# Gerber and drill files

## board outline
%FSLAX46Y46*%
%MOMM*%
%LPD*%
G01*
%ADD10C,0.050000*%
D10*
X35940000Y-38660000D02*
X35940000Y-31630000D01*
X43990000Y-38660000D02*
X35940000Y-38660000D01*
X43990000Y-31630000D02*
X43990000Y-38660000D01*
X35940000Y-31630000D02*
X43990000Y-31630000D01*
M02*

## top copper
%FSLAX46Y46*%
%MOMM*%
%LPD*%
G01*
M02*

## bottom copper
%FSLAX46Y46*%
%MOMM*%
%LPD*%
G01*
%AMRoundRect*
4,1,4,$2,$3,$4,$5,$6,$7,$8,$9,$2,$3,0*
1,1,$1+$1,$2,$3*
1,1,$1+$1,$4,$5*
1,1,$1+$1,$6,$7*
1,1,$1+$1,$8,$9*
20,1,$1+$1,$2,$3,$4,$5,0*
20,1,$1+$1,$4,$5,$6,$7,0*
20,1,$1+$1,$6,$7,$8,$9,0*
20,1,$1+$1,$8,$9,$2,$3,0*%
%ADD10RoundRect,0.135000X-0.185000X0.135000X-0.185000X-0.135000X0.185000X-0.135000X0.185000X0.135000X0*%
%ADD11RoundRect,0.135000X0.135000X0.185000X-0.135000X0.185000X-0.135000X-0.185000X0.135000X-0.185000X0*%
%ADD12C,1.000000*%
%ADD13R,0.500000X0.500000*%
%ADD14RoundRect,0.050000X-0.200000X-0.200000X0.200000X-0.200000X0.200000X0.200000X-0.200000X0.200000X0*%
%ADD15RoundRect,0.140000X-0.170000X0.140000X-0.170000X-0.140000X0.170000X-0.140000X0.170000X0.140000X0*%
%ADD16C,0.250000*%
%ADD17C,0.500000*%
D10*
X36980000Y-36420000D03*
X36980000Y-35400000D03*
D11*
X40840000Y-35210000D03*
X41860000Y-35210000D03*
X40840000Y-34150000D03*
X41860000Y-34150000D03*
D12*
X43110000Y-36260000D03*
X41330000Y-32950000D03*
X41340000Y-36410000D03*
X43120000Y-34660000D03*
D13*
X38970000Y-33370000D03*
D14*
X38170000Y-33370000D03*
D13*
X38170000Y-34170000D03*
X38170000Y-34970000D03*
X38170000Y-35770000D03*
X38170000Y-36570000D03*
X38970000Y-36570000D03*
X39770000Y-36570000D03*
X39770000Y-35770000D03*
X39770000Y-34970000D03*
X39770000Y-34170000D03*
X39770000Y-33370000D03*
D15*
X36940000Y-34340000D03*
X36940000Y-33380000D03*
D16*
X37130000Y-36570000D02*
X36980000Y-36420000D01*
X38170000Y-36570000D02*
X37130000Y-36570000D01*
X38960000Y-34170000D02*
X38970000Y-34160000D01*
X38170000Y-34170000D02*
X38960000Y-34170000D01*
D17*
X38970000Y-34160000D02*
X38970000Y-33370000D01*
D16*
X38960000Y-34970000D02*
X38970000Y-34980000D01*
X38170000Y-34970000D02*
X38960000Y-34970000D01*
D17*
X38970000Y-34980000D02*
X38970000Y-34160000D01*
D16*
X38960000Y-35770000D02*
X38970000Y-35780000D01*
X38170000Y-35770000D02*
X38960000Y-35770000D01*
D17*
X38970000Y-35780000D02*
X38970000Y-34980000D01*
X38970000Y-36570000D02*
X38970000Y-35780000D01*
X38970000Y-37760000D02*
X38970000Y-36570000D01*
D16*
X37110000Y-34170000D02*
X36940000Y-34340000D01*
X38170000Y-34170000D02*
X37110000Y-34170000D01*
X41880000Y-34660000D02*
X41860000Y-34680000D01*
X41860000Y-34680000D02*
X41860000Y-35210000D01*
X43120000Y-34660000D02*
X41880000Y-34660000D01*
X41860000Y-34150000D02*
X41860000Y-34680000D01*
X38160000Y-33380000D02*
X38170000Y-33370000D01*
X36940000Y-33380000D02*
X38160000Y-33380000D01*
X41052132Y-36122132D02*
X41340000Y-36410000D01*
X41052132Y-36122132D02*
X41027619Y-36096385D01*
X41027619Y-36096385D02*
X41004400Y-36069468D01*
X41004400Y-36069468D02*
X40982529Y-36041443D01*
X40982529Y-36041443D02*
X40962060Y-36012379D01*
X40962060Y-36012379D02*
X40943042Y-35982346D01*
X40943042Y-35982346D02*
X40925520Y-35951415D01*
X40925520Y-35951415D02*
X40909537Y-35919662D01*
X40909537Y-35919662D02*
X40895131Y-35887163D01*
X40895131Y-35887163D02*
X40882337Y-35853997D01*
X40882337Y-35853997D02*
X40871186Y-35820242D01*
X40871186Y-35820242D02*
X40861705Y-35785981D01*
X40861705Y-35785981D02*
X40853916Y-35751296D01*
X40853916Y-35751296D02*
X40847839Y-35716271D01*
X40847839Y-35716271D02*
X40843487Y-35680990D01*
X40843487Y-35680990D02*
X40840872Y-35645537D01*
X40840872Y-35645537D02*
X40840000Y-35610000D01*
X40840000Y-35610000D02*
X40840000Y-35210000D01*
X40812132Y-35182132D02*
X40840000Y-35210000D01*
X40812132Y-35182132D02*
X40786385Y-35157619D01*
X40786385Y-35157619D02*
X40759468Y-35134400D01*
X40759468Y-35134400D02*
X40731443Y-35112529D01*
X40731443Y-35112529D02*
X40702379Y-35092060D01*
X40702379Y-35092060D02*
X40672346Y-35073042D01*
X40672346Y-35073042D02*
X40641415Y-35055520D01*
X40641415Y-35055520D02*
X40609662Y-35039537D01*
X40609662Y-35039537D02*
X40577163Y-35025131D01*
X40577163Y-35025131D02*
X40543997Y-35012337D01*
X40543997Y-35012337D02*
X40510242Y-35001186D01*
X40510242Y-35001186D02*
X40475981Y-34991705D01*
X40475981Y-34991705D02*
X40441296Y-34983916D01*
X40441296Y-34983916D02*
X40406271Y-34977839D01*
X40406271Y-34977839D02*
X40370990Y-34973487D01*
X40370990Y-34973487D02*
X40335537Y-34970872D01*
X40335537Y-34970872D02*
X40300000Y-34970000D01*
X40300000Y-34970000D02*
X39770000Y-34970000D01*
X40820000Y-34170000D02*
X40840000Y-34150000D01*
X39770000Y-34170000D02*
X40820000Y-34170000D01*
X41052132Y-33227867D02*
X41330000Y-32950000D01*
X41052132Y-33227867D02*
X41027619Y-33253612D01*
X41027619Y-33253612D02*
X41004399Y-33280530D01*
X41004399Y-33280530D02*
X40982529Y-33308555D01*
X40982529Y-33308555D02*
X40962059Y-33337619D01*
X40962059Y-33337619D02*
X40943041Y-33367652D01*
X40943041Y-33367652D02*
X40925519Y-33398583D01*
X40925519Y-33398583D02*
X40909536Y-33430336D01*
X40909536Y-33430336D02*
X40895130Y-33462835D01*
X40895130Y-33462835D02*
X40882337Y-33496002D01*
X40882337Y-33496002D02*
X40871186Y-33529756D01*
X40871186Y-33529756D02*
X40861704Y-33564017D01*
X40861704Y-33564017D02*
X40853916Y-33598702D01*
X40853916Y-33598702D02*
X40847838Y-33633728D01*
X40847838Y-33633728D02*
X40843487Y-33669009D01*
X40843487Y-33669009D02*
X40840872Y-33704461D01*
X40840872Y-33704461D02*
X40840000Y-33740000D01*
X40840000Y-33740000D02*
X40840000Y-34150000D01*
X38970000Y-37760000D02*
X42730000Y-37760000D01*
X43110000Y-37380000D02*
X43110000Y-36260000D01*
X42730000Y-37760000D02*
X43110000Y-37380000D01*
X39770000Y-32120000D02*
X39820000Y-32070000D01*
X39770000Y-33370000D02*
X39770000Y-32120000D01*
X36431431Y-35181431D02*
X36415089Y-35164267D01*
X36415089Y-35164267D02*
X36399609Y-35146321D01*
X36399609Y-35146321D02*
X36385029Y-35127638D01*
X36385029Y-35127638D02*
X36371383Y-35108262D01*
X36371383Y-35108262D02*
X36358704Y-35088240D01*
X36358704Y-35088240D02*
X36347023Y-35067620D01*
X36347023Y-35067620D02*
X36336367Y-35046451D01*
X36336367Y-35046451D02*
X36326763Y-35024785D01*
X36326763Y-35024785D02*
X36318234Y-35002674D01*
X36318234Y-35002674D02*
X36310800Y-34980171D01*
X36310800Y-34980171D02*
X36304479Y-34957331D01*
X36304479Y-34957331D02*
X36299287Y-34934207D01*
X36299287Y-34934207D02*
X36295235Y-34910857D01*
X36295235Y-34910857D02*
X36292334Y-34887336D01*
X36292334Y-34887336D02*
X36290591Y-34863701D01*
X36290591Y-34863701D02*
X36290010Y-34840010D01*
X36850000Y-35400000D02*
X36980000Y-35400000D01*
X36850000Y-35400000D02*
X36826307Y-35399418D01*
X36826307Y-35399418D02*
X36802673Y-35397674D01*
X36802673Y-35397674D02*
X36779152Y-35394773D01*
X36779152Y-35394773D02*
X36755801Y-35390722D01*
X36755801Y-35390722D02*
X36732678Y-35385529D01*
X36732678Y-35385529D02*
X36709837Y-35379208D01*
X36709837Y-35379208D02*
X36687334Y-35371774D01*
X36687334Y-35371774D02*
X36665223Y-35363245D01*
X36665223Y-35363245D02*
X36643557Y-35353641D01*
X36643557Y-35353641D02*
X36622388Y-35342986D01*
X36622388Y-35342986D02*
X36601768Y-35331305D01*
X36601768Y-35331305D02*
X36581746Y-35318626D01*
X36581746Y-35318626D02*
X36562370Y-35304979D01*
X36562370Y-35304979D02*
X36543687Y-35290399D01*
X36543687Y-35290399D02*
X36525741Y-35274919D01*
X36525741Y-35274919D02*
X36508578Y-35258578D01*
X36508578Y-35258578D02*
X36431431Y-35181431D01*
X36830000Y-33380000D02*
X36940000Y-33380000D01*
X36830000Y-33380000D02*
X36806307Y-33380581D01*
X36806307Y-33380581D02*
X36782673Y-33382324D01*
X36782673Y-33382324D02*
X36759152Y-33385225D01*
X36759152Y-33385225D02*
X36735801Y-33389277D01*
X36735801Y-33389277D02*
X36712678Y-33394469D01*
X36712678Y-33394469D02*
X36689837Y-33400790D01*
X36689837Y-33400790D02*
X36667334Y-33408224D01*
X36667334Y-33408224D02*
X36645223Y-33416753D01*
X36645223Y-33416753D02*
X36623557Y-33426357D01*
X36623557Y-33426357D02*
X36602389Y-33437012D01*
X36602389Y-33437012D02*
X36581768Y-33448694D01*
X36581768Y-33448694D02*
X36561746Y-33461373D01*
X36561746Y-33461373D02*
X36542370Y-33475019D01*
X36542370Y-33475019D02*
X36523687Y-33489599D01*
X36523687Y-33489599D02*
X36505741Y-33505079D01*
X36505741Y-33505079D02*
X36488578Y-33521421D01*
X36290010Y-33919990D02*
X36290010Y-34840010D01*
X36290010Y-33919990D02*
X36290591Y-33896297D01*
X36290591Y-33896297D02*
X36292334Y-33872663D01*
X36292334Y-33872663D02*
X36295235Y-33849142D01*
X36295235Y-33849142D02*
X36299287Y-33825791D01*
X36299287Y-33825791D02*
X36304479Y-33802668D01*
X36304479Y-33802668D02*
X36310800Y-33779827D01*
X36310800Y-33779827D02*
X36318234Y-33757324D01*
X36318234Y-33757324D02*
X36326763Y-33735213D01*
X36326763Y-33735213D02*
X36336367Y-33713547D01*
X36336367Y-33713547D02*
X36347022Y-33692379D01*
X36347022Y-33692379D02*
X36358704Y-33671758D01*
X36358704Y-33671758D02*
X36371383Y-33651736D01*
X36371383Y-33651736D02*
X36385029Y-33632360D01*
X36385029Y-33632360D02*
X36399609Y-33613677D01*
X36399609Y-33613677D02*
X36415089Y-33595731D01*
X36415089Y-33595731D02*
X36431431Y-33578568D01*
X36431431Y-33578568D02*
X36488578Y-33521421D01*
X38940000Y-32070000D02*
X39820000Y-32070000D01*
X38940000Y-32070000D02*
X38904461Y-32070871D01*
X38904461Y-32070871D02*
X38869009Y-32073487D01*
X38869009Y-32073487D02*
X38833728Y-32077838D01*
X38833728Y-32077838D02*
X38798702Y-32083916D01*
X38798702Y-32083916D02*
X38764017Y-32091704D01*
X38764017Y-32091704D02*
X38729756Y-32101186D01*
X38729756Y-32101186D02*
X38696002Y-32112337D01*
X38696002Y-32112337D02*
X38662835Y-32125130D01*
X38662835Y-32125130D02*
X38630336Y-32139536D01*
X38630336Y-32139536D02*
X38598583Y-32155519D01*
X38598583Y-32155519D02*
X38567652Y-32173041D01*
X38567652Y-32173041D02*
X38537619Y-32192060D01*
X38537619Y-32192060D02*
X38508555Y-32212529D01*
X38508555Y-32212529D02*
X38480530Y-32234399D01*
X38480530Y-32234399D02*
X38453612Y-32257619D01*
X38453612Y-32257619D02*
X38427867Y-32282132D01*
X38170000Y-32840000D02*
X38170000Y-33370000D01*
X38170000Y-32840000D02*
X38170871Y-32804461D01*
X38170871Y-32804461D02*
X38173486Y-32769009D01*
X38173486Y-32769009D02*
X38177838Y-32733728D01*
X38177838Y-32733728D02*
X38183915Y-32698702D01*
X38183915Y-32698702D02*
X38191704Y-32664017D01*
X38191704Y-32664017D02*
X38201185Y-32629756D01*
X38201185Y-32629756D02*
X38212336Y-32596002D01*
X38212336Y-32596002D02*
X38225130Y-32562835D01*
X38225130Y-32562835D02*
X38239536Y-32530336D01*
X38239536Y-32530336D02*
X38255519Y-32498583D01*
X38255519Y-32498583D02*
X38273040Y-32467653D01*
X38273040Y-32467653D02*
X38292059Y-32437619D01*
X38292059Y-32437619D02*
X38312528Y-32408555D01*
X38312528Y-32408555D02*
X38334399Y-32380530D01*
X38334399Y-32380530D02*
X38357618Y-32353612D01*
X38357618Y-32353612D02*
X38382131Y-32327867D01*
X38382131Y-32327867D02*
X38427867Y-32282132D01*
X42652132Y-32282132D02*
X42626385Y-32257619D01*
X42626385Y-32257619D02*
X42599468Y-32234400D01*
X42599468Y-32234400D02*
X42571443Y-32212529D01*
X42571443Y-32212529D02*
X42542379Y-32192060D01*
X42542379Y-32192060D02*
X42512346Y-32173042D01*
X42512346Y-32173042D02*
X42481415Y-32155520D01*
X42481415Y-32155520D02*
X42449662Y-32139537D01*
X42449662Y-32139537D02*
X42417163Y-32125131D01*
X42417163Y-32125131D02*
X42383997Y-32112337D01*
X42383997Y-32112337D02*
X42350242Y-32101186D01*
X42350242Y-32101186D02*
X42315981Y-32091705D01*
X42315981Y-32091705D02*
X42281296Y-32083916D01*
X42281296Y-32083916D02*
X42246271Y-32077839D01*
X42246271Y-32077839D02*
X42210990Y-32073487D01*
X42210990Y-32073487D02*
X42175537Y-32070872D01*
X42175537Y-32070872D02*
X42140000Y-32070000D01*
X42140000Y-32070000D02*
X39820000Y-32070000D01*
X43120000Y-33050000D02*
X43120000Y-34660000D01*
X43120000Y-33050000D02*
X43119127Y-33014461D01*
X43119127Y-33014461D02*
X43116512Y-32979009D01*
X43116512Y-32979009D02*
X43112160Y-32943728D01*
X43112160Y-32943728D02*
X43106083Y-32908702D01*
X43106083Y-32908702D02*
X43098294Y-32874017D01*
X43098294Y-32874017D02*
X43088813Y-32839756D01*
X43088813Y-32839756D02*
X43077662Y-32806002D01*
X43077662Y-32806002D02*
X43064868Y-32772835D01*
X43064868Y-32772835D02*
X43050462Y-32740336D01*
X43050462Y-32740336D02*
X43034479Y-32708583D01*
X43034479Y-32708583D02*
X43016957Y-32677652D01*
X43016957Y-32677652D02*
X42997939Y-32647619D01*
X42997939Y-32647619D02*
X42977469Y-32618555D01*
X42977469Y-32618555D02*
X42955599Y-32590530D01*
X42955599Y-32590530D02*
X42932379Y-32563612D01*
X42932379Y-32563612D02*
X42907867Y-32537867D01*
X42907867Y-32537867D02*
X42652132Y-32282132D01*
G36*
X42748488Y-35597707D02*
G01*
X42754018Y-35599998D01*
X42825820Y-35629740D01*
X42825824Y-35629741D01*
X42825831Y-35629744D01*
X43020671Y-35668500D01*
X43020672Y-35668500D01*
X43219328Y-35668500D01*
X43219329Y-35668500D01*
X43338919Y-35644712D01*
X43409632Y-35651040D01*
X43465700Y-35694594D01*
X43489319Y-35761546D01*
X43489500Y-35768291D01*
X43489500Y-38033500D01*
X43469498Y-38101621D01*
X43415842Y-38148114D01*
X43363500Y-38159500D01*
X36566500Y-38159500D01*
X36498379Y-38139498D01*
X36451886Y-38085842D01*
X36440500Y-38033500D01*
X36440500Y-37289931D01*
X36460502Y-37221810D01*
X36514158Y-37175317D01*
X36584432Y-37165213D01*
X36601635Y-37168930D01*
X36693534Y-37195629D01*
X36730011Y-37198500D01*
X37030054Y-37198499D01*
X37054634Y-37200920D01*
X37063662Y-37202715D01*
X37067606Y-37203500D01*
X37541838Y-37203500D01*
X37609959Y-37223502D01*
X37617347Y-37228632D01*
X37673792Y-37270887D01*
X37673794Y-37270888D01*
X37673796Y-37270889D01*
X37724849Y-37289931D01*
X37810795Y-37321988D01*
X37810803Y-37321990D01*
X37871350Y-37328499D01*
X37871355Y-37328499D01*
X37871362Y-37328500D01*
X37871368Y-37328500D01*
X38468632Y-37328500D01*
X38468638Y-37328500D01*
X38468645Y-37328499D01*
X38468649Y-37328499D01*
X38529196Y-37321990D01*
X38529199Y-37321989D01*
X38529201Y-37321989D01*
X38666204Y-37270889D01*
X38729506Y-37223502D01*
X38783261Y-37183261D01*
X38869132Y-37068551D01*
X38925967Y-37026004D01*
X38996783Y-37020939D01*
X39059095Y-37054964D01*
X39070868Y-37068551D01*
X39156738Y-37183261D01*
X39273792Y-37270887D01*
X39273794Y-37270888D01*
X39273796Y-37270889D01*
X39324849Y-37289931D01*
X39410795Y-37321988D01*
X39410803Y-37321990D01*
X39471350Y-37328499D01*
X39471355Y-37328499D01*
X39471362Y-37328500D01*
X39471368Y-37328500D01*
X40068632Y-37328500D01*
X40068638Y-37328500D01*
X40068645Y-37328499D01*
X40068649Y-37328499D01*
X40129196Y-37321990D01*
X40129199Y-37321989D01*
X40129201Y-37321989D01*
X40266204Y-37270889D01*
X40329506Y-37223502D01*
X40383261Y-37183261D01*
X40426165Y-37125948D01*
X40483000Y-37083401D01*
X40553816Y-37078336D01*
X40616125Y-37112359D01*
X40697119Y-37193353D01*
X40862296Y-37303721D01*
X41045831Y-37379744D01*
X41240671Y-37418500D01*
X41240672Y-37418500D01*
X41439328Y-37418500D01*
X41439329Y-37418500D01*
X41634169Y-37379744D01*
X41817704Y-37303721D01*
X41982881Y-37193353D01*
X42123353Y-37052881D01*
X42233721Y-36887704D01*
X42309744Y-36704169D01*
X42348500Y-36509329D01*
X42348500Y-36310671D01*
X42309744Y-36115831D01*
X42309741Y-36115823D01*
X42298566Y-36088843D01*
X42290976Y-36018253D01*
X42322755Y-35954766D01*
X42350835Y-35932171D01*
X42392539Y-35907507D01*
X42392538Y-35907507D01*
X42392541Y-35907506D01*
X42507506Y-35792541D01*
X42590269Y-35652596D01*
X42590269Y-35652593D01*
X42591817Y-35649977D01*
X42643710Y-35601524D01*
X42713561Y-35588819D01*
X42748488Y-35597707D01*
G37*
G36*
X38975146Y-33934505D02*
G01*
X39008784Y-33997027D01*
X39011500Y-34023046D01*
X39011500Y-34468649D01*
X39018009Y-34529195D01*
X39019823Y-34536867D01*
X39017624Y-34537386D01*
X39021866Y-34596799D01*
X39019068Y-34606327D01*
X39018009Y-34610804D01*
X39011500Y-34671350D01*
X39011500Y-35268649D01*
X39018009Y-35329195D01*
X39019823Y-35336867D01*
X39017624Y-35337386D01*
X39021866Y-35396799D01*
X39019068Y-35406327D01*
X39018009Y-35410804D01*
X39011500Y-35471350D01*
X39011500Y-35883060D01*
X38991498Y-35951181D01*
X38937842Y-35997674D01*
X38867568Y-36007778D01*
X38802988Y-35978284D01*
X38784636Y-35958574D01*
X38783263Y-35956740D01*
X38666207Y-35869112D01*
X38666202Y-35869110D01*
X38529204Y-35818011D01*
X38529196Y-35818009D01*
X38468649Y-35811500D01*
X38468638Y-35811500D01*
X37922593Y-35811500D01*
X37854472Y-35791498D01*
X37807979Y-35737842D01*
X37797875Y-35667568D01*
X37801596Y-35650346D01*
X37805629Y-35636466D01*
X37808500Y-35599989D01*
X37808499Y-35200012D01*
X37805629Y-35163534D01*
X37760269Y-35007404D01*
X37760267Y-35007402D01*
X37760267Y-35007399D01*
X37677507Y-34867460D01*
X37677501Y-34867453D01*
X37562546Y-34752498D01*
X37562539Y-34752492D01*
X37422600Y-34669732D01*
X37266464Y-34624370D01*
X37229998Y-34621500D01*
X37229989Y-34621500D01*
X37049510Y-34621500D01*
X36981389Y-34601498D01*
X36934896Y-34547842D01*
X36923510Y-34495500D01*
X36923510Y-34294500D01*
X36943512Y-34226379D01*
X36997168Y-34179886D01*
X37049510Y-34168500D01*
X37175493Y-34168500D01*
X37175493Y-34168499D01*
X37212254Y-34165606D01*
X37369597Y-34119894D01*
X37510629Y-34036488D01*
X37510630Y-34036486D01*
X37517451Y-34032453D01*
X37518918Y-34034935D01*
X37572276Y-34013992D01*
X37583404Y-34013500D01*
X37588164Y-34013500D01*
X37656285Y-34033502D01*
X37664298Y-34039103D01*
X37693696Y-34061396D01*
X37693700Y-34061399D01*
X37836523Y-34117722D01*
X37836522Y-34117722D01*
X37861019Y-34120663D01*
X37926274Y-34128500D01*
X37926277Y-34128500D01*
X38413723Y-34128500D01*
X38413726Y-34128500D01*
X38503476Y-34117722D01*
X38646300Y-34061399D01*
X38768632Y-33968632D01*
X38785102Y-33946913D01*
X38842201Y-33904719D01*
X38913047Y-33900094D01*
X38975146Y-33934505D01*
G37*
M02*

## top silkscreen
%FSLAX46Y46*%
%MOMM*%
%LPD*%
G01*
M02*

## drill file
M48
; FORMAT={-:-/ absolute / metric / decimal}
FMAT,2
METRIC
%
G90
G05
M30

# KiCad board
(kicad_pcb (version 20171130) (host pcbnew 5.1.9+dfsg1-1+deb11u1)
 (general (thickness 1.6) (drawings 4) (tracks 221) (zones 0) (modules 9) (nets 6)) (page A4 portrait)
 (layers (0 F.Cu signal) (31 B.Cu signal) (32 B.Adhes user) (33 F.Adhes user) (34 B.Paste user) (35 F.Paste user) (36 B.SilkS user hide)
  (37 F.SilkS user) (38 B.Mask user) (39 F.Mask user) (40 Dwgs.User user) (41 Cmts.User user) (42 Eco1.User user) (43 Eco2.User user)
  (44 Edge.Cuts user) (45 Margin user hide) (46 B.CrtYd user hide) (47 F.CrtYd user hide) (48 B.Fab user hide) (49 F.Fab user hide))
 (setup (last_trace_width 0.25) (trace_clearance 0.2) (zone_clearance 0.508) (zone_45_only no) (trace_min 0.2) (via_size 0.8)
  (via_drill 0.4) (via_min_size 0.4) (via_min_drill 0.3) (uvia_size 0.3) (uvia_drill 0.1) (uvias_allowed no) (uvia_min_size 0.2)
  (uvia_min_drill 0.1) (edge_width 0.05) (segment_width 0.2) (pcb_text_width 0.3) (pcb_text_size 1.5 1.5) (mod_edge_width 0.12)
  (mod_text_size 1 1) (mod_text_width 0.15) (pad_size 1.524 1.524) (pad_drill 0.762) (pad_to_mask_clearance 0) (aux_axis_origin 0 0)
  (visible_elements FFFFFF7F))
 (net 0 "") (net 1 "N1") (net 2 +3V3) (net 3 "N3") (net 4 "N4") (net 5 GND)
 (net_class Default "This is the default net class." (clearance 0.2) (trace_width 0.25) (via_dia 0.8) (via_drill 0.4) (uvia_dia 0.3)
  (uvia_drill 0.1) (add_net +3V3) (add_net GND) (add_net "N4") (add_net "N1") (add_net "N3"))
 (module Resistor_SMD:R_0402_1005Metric (layer B.Cu) (at 36.98 35.91 270)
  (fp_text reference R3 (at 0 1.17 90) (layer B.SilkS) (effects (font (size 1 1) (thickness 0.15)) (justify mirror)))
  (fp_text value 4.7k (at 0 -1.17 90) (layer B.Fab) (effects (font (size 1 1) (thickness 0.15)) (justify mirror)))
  (pad 2 smd roundrect (at 0.51 0 270) (size 0.54 0.64) (layers B.Cu B.Paste B.Mask) (roundrect_rratio 0.25) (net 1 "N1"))
  (pad 1 smd roundrect (at -0.51 0 270) (size 0.54 0.64) (layers B.Cu B.Paste B.Mask) (roundrect_rratio 0.25) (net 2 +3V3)))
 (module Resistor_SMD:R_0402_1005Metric (layer B.Cu) (at 41.35 35.21 180)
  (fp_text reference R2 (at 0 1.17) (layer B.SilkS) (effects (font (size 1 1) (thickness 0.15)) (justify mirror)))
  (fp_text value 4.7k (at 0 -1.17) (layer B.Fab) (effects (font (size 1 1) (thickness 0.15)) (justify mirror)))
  (pad 2 smd roundrect (at 0.51 0 180) (size 0.54 0.64) (layers B.Cu B.Paste B.Mask) (roundrect_rratio 0.25) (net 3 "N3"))
  (pad 1 smd roundrect (at -0.51 0 180) (size 0.54 0.64) (layers B.Cu B.Paste B.Mask) (roundrect_rratio 0.25) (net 2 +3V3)))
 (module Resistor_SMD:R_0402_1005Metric (layer B.Cu) (at 41.35 34.15 180)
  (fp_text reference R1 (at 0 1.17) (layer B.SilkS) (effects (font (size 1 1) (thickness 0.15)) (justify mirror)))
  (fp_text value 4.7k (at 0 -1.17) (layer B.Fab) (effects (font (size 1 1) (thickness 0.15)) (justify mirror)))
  (pad 2 smd roundrect (at 0.51 0 180) (size 0.54 0.64) (layers B.Cu B.Paste B.Mask) (roundrect_rratio 0.25) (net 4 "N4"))
  (pad 1 smd roundrect (at -0.51 0 180) (size 0.54 0.64) (layers B.Cu B.Paste B.Mask) (roundrect_rratio 0.25) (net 2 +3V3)))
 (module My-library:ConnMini (layer B.Cu) (at 43.11 36.26)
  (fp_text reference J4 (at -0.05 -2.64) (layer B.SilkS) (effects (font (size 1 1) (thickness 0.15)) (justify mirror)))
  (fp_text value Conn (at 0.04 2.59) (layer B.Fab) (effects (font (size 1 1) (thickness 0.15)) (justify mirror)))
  (pad 1 smd circle (at 0 0) (size 1 1) (layers B.Cu B.Paste B.Mask) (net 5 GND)))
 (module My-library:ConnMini (layer B.Cu) (at 41.33 32.95)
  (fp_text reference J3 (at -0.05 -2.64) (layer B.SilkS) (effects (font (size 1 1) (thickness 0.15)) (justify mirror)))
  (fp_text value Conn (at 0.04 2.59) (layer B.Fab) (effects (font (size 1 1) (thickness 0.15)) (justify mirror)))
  (pad 1 smd circle (at 0 0) (size 1 1) (layers B.Cu B.Paste B.Mask) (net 4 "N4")))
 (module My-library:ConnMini (layer B.Cu) (at 41.34 36.41)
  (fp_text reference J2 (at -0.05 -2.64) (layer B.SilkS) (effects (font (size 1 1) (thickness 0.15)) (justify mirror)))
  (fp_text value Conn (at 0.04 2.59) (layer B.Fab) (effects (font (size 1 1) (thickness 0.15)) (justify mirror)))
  (pad 1 smd circle (at 0 0) (size 1 1) (layers B.Cu B.Paste B.Mask) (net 3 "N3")))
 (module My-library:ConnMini (layer B.Cu) (at 43.12 34.66)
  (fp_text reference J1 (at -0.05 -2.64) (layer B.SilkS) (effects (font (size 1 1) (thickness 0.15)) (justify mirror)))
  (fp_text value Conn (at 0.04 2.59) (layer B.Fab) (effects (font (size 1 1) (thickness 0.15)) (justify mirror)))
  (pad 1 smd circle (at 0 0) (size 1 1) (layers B.Cu B.Paste B.Mask) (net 2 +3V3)))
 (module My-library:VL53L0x (layer B.Cu) (at 38.97 34.97)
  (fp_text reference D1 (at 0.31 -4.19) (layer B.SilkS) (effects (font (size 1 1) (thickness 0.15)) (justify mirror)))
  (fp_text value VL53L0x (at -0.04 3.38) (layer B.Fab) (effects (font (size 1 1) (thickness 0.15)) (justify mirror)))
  (pad 12 smd rect (at 0 -1.6) (size 0.5 0.5) (layers B.Cu B.Paste B.Mask) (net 5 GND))
  (pad 1 smd roundrect (at -0.8 -1.6) (size 0.5 0.5) (layers B.Cu B.Paste B.Mask) (roundrect_rratio 0.1) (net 2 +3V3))
  (pad 2 smd rect (at -0.8 -0.8) (size 0.5 0.5) (layers B.Cu B.Paste B.Mask) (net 5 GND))
  (pad 3 smd rect (at -0.8 0) (size 0.5 0.5) (layers B.Cu B.Paste B.Mask) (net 5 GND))
  (pad 4 smd rect (at -0.8 0.8) (size 0.5 0.5) (layers B.Cu B.Paste B.Mask) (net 5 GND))
  (pad 5 smd rect (at -0.8 1.6) (size 0.5 0.5) (layers B.Cu B.Paste B.Mask) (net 1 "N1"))
  (pad 6 smd rect (at 0 1.6) (size 0.5 0.5) (layers B.Cu B.Paste B.Mask) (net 5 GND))
  (pad 7 smd rect (at 0.8 1.6) (size 0.5 0.5) (layers B.Cu B.Paste B.Mask))
  (pad 8 smd rect (at 0.8 0.8) (size 0.5 0.5) (layers B.Cu B.Paste B.Mask))
  (pad 9 smd rect (at 0.8 0) (size 0.5 0.5) (layers B.Cu B.Paste B.Mask) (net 3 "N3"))
  (pad 10 smd rect (at 0.8 -0.8) (size 0.5 0.5) (layers B.Cu B.Paste B.Mask) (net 4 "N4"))
  (pad 11 smd rect (at 0.8 -1.6) (size 0.5 0.5) (layers B.Cu B.Paste B.Mask) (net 2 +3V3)))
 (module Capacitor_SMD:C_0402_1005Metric (layer B.Cu) (at 36.94 33.86 270)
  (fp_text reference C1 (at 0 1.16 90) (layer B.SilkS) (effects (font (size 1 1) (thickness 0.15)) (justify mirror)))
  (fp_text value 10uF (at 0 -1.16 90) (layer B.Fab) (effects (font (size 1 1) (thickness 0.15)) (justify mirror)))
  (pad 2 smd roundrect (at 0.48 0 270) (size 0.56 0.62) (layers B.Cu B.Paste B.Mask) (roundrect_rratio 0.25) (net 5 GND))
  (pad 1 smd roundrect (at -0.48 0 270) (size 0.56 0.62) (layers B.Cu B.Paste B.Mask) (roundrect_rratio 0.25) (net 2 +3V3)))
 (gr_line (start 35.94 38.66) (end 35.94 31.63) (layer Edge.Cuts) (width 0.05))
 (gr_line (start 43.99 38.66) (end 35.94 38.66) (layer Edge.Cuts) (width 0.05))
 (gr_line (start 43.99 31.63) (end 43.99 38.66) (layer Edge.Cuts) (width 0.05))
 (gr_line (start 35.94 31.63) (end 43.99 31.63) (layer Edge.Cuts) (width 0.05))
 (segment (start 37.13 36.57) (end 36.98 36.42) (width 0.25) (layer B.Cu) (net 1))
 (segment (start 38.17 36.57) (end 37.13 36.57) (width 0.25) (layer B.Cu) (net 1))
 (segment (start 38.96 34.17) (end 38.97 34.16) (width 0.25) (layer B.Cu) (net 5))
 (segment (start 38.17 34.17) (end 38.96 34.17) (width 0.25) (layer B.Cu) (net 5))
 (segment (start 38.97 34.16) (end 38.97 33.37) (width 0.5) (layer B.Cu) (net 5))
 (segment (start 38.96 34.97) (end 38.97 34.98) (width 0.25) (layer B.Cu) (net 5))
 (segment (start 38.17 34.97) (end 38.96 34.97) (width 0.25) (layer B.Cu) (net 5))
 (segment (start 38.97 34.98) (end 38.97 34.16) (width 0.5) (layer B.Cu) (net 5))
 (segment (start 38.96 35.77) (end 38.97 35.78) (width 0.25) (layer B.Cu) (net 5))
 (segment (start 38.17 35.77) (end 38.96 35.77) (width 0.25) (layer B.Cu) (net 5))
 (segment (start 38.97 35.78) (end 38.97 34.98) (width 0.5) (layer B.Cu) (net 5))
 (segment (start 38.97 36.57) (end 38.97 35.78) (width 0.5) (layer B.Cu) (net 5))
 (segment (start 38.97 37.76) (end 38.97 36.57) (width 0.5) (layer B.Cu) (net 5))
 (segment (start 37.11 34.17) (end 36.94 34.34) (width 0.25) (layer B.Cu) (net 5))
 (segment (start 38.17 34.17) (end 37.11 34.17) (width 0.25) (layer B.Cu) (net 5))
 (segment (start 41.88 34.66) (end 41.86 34.68) (width 0.25) (layer B.Cu) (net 2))
 (segment (start 41.86 34.68) (end 41.86 35.21) (width 0.25) (layer B.Cu) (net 2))
 (segment (start 43.12 34.66) (end 41.88 34.66) (width 0.25) (layer B.Cu) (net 2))
 (segment (start 41.86 34.15) (end 41.86 34.68) (width 0.25) (layer B.Cu) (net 2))
 (segment (start 38.16 33.38) (end 38.17 33.37) (width 0.25) (layer B.Cu) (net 2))
 (segment (start 36.94 33.38) (end 38.16 33.38) (width 0.25) (layer B.Cu) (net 2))
 (segment (start 41.052132 36.122132) (end 41.34 36.41) (width 0.25) (layer B.Cu) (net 3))
 (segment (start 41.052132 36.122132) (end 41.027619 36.096385) (width 0.25) (layer B.Cu) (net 3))
 (segment (start 41.027619 36.096385) (end 41.0044 36.069468) (width 0.25) (layer B.Cu) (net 3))
 (segment (start 41.0044 36.069468) (end 40.982529 36.041443) (width 0.25) (layer B.Cu) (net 3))
 (segment (start 40.982529 36.041443) (end 40.96206 36.012379) (width 0.25) (layer B.Cu) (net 3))
 (segment (start 40.96206 36.012379) (end 40.943042 35.982346) (width 0.25) (layer B.Cu) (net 3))
 (segment (start 40.943042 35.982346) (end 40.92552 35.951415) (width 0.25) (layer B.Cu) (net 3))
 (segment (start 40.92552 35.951415) (end 40.909537 35.919662) (width 0.25) (layer B.Cu) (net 3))
 (segment (start 40.909537 35.919662) (end 40.895131 35.887163) (width 0.25) (layer B.Cu) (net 3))
 (segment (start 40.895131 35.887163) (end 40.882337 35.853997) (width 0.25) (layer B.Cu) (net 3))
 (segment (start 40.882337 35.853997) (end 40.871186 35.820242) (width 0.25) (layer B.Cu) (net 3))
 (segment (start 40.871186 35.820242) (end 40.861705 35.785981) (width 0.25) (layer B.Cu) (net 3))
 (segment (start 40.861705 35.785981) (end 40.853916 35.751296) (width 0.25) (layer B.Cu) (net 3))
 (segment (start 40.853916 35.751296) (end 40.847839 35.716271) (width 0.25) (layer B.Cu) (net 3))
 (segment (start 40.847839 35.716271) (end 40.843487 35.68099) (width 0.25) (layer B.Cu) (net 3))
 (segment (start 40.843487 35.68099) (end 40.840872 35.645537) (width 0.25) (layer B.Cu) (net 3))
 (segment (start 40.840872 35.645537) (end 40.84 35.61) (width 0.25) (layer B.Cu) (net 3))
 (segment (start 40.84 35.61) (end 40.84 35.21) (width 0.25) (layer B.Cu) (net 3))
 (segment (start 40.812132 35.182132) (end 40.84 35.21) (width 0.25) (layer B.Cu) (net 3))
 (segment (start 40.812132 35.182132) (end 40.786385 35.157619) (width 0.25) (layer B.Cu) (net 3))
 (segment (start 40.786385 35.157619) (end 40.759468 35.1344) (width 0.25) (layer B.Cu) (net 3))
 (segment (start 40.759468 35.1344) (end 40.731443 35.112529) (width 0.25) (layer B.Cu) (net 3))
 (segment (start 40.731443 35.112529) (end 40.702379 35.09206) (width 0.25) (layer B.Cu) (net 3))
 (segment (start 40.702379 35.09206) (end 40.672346 35.073042) (width 0.25) (layer B.Cu) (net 3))
 (segment (start 40.672346 35.073042) (end 40.641415 35.05552) (width 0.25) (layer B.Cu) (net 3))
 (segment (start 40.641415 35.05552) (end 40.609662 35.039537) (width 0.25) (layer B.Cu) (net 3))
 (segment (start 40.609662 35.039537) (end 40.577163 35.025131) (width 0.25) (layer B.Cu) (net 3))
 (segment (start 40.577163 35.025131) (end 40.543997 35.012337) (width 0.25) (layer B.Cu) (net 3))
 (segment (start 40.543997 35.012337) (end 40.510242 35.001186) (width 0.25) (layer B.Cu) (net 3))
 (segment (start 40.510242 35.001186) (end 40.475981 34.991705) (width 0.25) (layer B.Cu) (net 3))
 (segment (start 40.475981 34.991705) (end 40.441296 34.983916) (width 0.25) (layer B.Cu) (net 3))
 (segment (start 40.441296 34.983916) (end 40.406271 34.977839) (width 0.25) (layer B.Cu) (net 3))
 (segment (start 40.406271 34.977839) (end 40.37099 34.973487) (width 0.25) (layer B.Cu) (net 3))
 (segment (start 40.37099 34.973487) (end 40.335537 34.970872) (width 0.25) (layer B.Cu) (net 3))
 (segment (start 40.335537 34.970872) (end 40.3 34.97) (width 0.25) (layer B.Cu) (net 3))
 (segment (start 40.3 34.97) (end 39.77 34.97) (width 0.25) (layer B.Cu) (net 3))
 (segment (start 40.82 34.17) (end 40.84 34.15) (width 0.25) (layer B.Cu) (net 4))
 (segment (start 39.77 34.17) (end 40.82 34.17) (width 0.25) (layer B.Cu) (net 4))
 (segment (start 41.052132 33.227867) (end 41.33 32.95) (width 0.25) (layer B.Cu) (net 4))
 (segment (start 41.052132 33.227867) (end 41.027619 33.253612) (width 0.25) (layer B.Cu) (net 4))
 (segment (start 41.027619 33.253612) (end 41.004399 33.28053) (width 0.25) (layer B.Cu) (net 4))
 (segment (start 41.004399 33.28053) (end 40.982529 33.308555) (width 0.25) (layer B.Cu) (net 4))
 (segment (start 40.982529 33.308555) (end 40.962059 33.337619) (width 0.25) (layer B.Cu) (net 4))
 (segment (start 40.962059 33.337619) (end 40.943041 33.367652) (width 0.25) (layer B.Cu) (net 4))
 (segment (start 40.943041 33.367652) (end 40.925519 33.398583) (width 0.25) (layer B.Cu) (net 4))
 (segment (start 40.925519 33.398583) (end 40.909536 33.430336) (width 0.25) (layer B.Cu) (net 4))
 (segment (start 40.909536 33.430336) (end 40.89513 33.462835) (width 0.25) (layer B.Cu) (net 4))
 (segment (start 40.89513 33.462835) (end 40.882337 33.496002) (width 0.25) (layer B.Cu) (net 4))
 (segment (start 40.882337 33.496002) (end 40.871186 33.529756) (width 0.25) (layer B.Cu) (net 4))
 (segment (start 40.871186 33.529756) (end 40.861704 33.564017) (width 0.25) (layer B.Cu) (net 4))
 (segment (start 40.861704 33.564017) (end 40.853916 33.598702) (width 0.25) (layer B.Cu) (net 4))
 (segment (start 40.853916 33.598702) (end 40.847838 33.633728) (width 0.25) (layer B.Cu) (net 4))
 (segment (start 40.847838 33.633728) (end 40.843487 33.669009) (width 0.25) (layer B.Cu) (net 4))
 (segment (start 40.843487 33.669009) (end 40.840872 33.704461) (width 0.25) (layer B.Cu) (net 4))
 (segment (start 40.840872 33.704461) (end 40.84 33.74) (width 0.25) (layer B.Cu) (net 4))
 (segment (start 40.84 33.74) (end 40.84 34.15) (width 0.25) (layer B.Cu) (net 4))
 (segment (start 38.97 37.76) (end 42.73 37.76) (width 0.25) (layer B.Cu) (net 5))
 (segment (start 43.11 37.38) (end 43.11 36.26) (width 0.25) (layer B.Cu) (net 5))
 (segment (start 42.73 37.76) (end 43.11 37.38) (width 0.25) (layer B.Cu) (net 5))
 (segment (start 39.77 32.12) (end 39.82 32.07) (width 0.25) (layer B.Cu) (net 2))
 (segment (start 39.77 33.37) (end 39.77 32.12) (width 0.25) (layer B.Cu) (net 2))
 (segment (start 36.431431 35.181431) (end 36.415089 35.164267) (width 0.25) (layer B.Cu) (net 2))
 (segment (start 36.415089 35.164267) (end 36.399609 35.146321) (width 0.25) (layer B.Cu) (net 2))
 (segment (start 36.399609 35.146321) (end 36.385029 35.127638) (width 0.25) (layer B.Cu) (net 2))
 (segment (start 36.385029 35.127638) (end 36.371383 35.108262) (width 0.25) (layer B.Cu) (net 2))
 (segment (start 36.371383 35.108262) (end 36.358704 35.08824) (width 0.25) (layer B.Cu) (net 2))
 (segment (start 36.358704 35.08824) (end 36.347023 35.06762) (width 0.25) (layer B.Cu) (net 2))
 (segment (start 36.347023 35.06762) (end 36.336367 35.046451) (width 0.25) (layer B.Cu) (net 2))
 (segment (start 36.336367 35.046451) (end 36.326763 35.024785) (width 0.25) (layer B.Cu) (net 2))
 (segment (start 36.326763 35.024785) (end 36.318234 35.002674) (width 0.25) (layer B.Cu) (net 2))
 (segment (start 36.318234 35.002674) (end 36.3108 34.980171) (width 0.25) (layer B.Cu) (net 2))
 (segment (start 36.3108 34.980171) (end 36.304479 34.957331) (width 0.25) (layer B.Cu) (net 2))
 (segment (start 36.304479 34.957331) (end 36.299287 34.934207) (width 0.25) (layer B.Cu) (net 2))
 (segment (start 36.299287 34.934207) (end 36.295235 34.910857) (width 0.25) (layer B.Cu) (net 2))
 (segment (start 36.295235 34.910857) (end 36.292334 34.887336) (width 0.25) (layer B.Cu) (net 2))
 (segment (start 36.292334 34.887336) (end 36.290591 34.863701) (width 0.25) (layer B.Cu) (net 2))
 (segment (start 36.290591 34.863701) (end 36.29001 34.84001) (width 0.25) (layer B.Cu) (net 2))
 (segment (start 36.85 35.4) (end 36.98 35.4) (width 0.25) (layer B.Cu) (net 2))
 (segment (start 36.85 35.4) (end 36.826307 35.399418) (width 0.25) (layer B.Cu) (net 2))
 (segment (start 36.826307 35.399418) (end 36.802673 35.397674) (width 0.25) (layer B.Cu) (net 2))
 (segment (start 36.802673 35.397674) (end 36.779152 35.394773) (width 0.25) (layer B.Cu) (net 2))
 (segment (start 36.779152 35.394773) (end 36.755801 35.390722) (width 0.25) (layer B.Cu) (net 2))
 (segment (start 36.755801 35.390722) (end 36.732678 35.385529) (width 0.25) (layer B.Cu) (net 2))
 (segment (start 36.732678 35.385529) (end 36.709837 35.379208) (width 0.25) (layer B.Cu) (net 2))
 (segment (start 36.709837 35.379208) (end 36.687334 35.371774) (width 0.25) (layer B.Cu) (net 2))
 (segment (start 36.687334 35.371774) (end 36.665223 35.363245) (width 0.25) (layer B.Cu) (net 2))
 (segment (start 36.665223 35.363245) (end 36.643557 35.353641) (width 0.25) (layer B.Cu) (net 2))
 (segment (start 36.643557 35.353641) (end 36.622388 35.342986) (width 0.25) (layer B.Cu) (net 2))
 (segment (start 36.622388 35.342986) (end 36.601768 35.331305) (width 0.25) (layer B.Cu) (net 2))
 (segment (start 36.601768 35.331305) (end 36.581746 35.318626) (width 0.25) (layer B.Cu) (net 2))
 (segment (start 36.581746 35.318626) (end 36.56237 35.304979) (width 0.25) (layer B.Cu) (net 2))
 (segment (start 36.56237 35.304979) (end 36.543687 35.290399) (width 0.25) (layer B.Cu) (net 2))
 (segment (start 36.543687 35.290399) (end 36.525741 35.274919) (width 0.25) (layer B.Cu) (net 2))
 (segment (start 36.525741 35.274919) (end 36.508578 35.258578) (width 0.25) (layer B.Cu) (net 2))
 (segment (start 36.508578 35.258578) (end 36.431431 35.181431) (width 0.25) (layer B.Cu) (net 2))
 (segment (start 36.83 33.38) (end 36.94 33.38) (width 0.25) (layer B.Cu) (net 2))
 (segment (start 36.83 33.38) (end 36.806307 33.380581) (width 0.25) (layer B.Cu) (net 2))
 (segment (start 36.806307 33.380581) (end 36.782673 33.382324) (width 0.25) (layer B.Cu) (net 2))
 (segment (start 36.782673 33.382324) (end 36.759152 33.385225) (width 0.25) (layer B.Cu) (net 2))
 (segment (start 36.759152 33.385225) (end 36.735801 33.389277) (width 0.25) (layer B.Cu) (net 2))
 (segment (start 36.735801 33.389277) (end 36.712678 33.394469) (width 0.25) (layer B.Cu) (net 2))
 (segment (start 36.712678 33.394469) (end 36.689837 33.40079) (width 0.25) (layer B.Cu) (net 2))
 (segment (start 36.689837 33.40079) (end 36.667334 33.408224) (width 0.25) (layer B.Cu) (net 2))
 (segment (start 36.667334 33.408224) (end 36.645223 33.416753) (width 0.25) (layer B.Cu) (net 2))
 (segment (start 36.645223 33.416753) (end 36.623557 33.426357) (width 0.25) (layer B.Cu) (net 2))
 (segment (start 36.623557 33.426357) (end 36.602389 33.437012) (width 0.25) (layer B.Cu) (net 2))
 (segment (start 36.602389 33.437012) (end 36.581768 33.448694) (width 0.25) (layer B.Cu) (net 2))
 (segment (start 36.581768 33.448694) (end 36.561746 33.461373) (width 0.25) (layer B.Cu) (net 2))
 (segment (start 36.561746 33.461373) (end 36.54237 33.475019) (width 0.25) (layer B.Cu) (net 2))
 (segment (start 36.54237 33.475019) (end 36.523687 33.489599) (width 0.25) (layer B.Cu) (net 2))
 (segment (start 36.523687 33.489599) (end 36.505741 33.505079) (width 0.25) (layer B.Cu) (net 2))
 (segment (start 36.505741 33.505079) (end 36.488578 33.521421) (width 0.25) (layer B.Cu) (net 2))
 (segment (start 36.29001 33.91999) (end 36.29001 34.84001) (width 0.25) (layer B.Cu) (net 2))
 (segment (start 36.29001 33.91999) (end 36.290591 33.896297) (width 0.25) (layer B.Cu) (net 2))
 (segment (start 36.290591 33.896297) (end 36.292334 33.872663) (width 0.25) (layer B.Cu) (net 2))
 (segment (start 36.292334 33.872663) (end 36.295235 33.849142) (width 0.25) (layer B.Cu) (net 2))
 (segment (start 36.295235 33.849142) (end 36.299287 33.825791) (width 0.25) (layer B.Cu) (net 2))
 (segment (start 36.299287 33.825791) (end 36.304479 33.802668) (width 0.25) (layer B.Cu) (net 2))
 (segment (start 36.304479 33.802668) (end 36.3108 33.779827) (width 0.25) (layer B.Cu) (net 2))
 (segment (start 36.3108 33.779827) (end 36.318234 33.757324) (width 0.25) (layer B.Cu) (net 2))
 (segment (start 36.318234 33.757324) (end 36.326763 33.735213) (width 0.25) (layer B.Cu) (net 2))
 (segment (start 36.326763 33.735213) (end 36.336367 33.713547) (width 0.25) (layer B.Cu) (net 2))
 (segment (start 36.336367 33.713547) (end 36.347022 33.692379) (width 0.25) (layer B.Cu) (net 2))
 (segment (start 36.347022 33.692379) (end 36.358704 33.671758) (width 0.25) (layer B.Cu) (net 2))
 (segment (start 36.358704 33.671758) (end 36.371383 33.651736) (width 0.25) (layer B.Cu) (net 2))
 (segment (start 36.371383 33.651736) (end 36.385029 33.63236) (width 0.25) (layer B.Cu) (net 2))
 (segment (start 36.385029 33.63236) (end 36.399609 33.613677) (width 0.25) (layer B.Cu) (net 2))
 (segment (start 36.399609 33.613677) (end 36.415089 33.595731) (width 0.25) (layer B.Cu) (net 2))
 (segment (start 36.415089 33.595731) (end 36.431431 33.578568) (width 0.25) (layer B.Cu) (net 2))
 (segment (start 36.431431 33.578568) (end 36.488578 33.521421) (width 0.25) (layer B.Cu) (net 2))
 (segment (start 38.94 32.07) (end 39.82 32.07) (width 0.25) (layer B.Cu) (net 2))
 (segment (start 38.94 32.07) (end 38.904461 32.070871) (width 0.25) (layer B.Cu) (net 2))
 (segment (start 38.904461 32.070871) (end 38.869009 32.073487) (width 0.25) (layer B.Cu) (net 2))
 (segment (start 38.869009 32.073487) (end 38.833728 32.077838) (width 0.25) (layer B.Cu) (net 2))
 (segment (start 38.833728 32.077838) (end 38.798702 32.083916) (width 0.25) (layer B.Cu) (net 2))
 (segment (start 38.798702 32.083916) (end 38.764017 32.091704) (width 0.25) (layer B.Cu) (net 2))
 (segment (start 38.764017 32.091704) (end 38.729756 32.101186) (width 0.25) (layer B.Cu) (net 2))
 (segment (start 38.729756 32.101186) (end 38.696002 32.112337) (width 0.25) (layer B.Cu) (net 2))
 (segment (start 38.696002 32.112337) (end 38.662835 32.12513) (width 0.25) (layer B.Cu) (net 2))
 (segment (start 38.662835 32.12513) (end 38.630336 32.139536) (width 0.25) (layer B.Cu) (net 2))
 (segment (start 38.630336 32.139536) (end 38.598583 32.155519) (width 0.25) (layer B.Cu) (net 2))
 (segment (start 38.598583 32.155519) (end 38.567652 32.173041) (width 0.25) (layer B.Cu) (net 2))
 (segment (start 38.567652 32.173041) (end 38.537619 32.19206) (width 0.25) (layer B.Cu) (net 2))
 (segment (start 38.537619 32.19206) (end 38.508555 32.212529) (width 0.25) (layer B.Cu) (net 2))
 (segment (start 38.508555 32.212529) (end 38.48053 32.234399) (width 0.25) (layer B.Cu) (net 2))
 (segment (start 38.48053 32.234399) (end 38.453612 32.257619) (width 0.25) (layer B.Cu) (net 2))
 (segment (start 38.453612 32.257619) (end 38.427867 32.282132) (width 0.25) (layer B.Cu) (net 2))
 (segment (start 38.17 32.84) (end 38.17 33.37) (width 0.25) (layer B.Cu) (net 2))
 (segment (start 38.17 32.84) (end 38.170871 32.804461) (width 0.25) (layer B.Cu) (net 2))
 (segment (start 38.170871 32.804461) (end 38.173486 32.769009) (width 0.25) (layer B.Cu) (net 2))
 (segment (start 38.173486 32.769009) (end 38.177838 32.733728) (width 0.25) (layer B.Cu) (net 2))
 (segment (start 38.177838 32.733728) (end 38.183915 32.698702) (width 0.25) (layer B.Cu) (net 2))
 (segment (start 38.183915 32.698702) (end 38.191704 32.664017) (width 0.25) (layer B.Cu) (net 2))
 (segment (start 38.191704 32.664017) (end 38.201185 32.629756) (width 0.25) (layer B.Cu) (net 2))
 (segment (start 38.201185 32.629756) (end 38.212336 32.596002) (width 0.25) (layer B.Cu) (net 2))
 (segment (start 38.212336 32.596002) (end 38.22513 32.562835) (width 0.25) (layer B.Cu) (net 2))
 (segment (start 38.22513 32.562835) (end 38.239536 32.530336) (width 0.25) (layer B.Cu) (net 2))
 (segment (start 38.239536 32.530336) (end 38.255519 32.498583) (width 0.25) (layer B.Cu) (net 2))
 (segment (start 38.255519 32.498583) (end 38.27304 32.467653) (width 0.25) (layer B.Cu) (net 2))
 (segment (start 38.27304 32.467653) (end 38.292059 32.437619) (width 0.25) (layer B.Cu) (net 2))
 (segment (start 38.292059 32.437619) (end 38.312528 32.408555) (width 0.25) (layer B.Cu) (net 2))
 (segment (start 38.312528 32.408555) (end 38.334399 32.38053) (width 0.25) (layer B.Cu) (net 2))
 (segment (start 38.334399 32.38053) (end 38.357618 32.353612) (width 0.25) (layer B.Cu) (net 2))
 (segment (start 38.357618 32.353612) (end 38.382131 32.327867) (width 0.25) (layer B.Cu) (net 2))
 (segment (start 38.382131 32.327867) (end 38.427867 32.282132) (width 0.25) (layer B.Cu) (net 2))
 (segment (start 42.652132 32.282132) (end 42.626385 32.257619) (width 0.25) (layer B.Cu) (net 2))
 (segment (start 42.626385 32.257619) (end 42.599468 32.2344) (width 0.25) (layer B.Cu) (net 2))
 (segment (start 42.599468 32.2344) (end 42.571443 32.212529) (width 0.25) (layer B.Cu) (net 2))
 (segment (start 42.571443 32.212529) (end 42.542379 32.19206) (width 0.25) (layer B.Cu) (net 2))
 (segment (start 42.542379 32.19206) (end 42.512346 32.173042) (width 0.25) (layer B.Cu) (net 2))
 (segment (start 42.512346 32.173042) (end 42.481415 32.15552) (width 0.25) (layer B.Cu) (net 2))
 (segment (start 42.481415 32.15552) (end 42.449662 32.139537) (width 0.25) (layer B.Cu) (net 2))
 (segment (start 42.449662 32.139537) (end 42.417163 32.125131) (width 0.25) (layer B.Cu) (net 2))
 (segment (start 42.417163 32.125131) (end 42.383997 32.112337) (width 0.25) (layer B.Cu) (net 2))
 (segment (start 42.383997 32.112337) (end 42.350242 32.101186) (width 0.25) (layer B.Cu) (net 2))
 (segment (start 42.350242 32.101186) (end 42.315981 32.091705) (width 0.25) (layer B.Cu) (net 2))
 (segment (start 42.315981 32.091705) (end 42.281296 32.083916) (width 0.25) (layer B.Cu) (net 2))
 (segment (start 42.281296 32.083916) (end 42.246271 32.077839) (width 0.25) (layer B.Cu) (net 2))
 (segment (start 42.246271 32.077839) (end 42.21099 32.073487) (width 0.25) (layer B.Cu) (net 2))
 (segment (start 42.21099 32.073487) (end 42.175537 32.070872) (width 0.25) (layer B.Cu) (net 2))
 (segment (start 42.175537 32.070872) (end 42.14 32.07) (width 0.25) (layer B.Cu) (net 2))
 (segment (start 42.14 32.07) (end 39.82 32.07) (width 0.25) (layer B.Cu) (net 2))
 (segment (start 43.12 33.05) (end 43.12 34.66) (width 0.25) (layer B.Cu) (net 2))
 (segment (start 43.12 33.05) (end 43.119127 33.014461) (width 0.25) (layer B.Cu) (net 2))
 (segment (start 43.119127 33.014461) (end 43.116512 32.979009) (width 0.25) (layer B.Cu) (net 2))
 (segment (start 43.116512 32.979009) (end 43.11216 32.943728) (width 0.25) (layer B.Cu) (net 2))
 (segment (start 43.11216 32.943728) (end 43.106083 32.908702) (width 0.25) (layer B.Cu) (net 2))
 (segment (start 43.106083 32.908702) (end 43.098294 32.874017) (width 0.25) (layer B.Cu) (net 2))
 (segment (start 43.098294 32.874017) (end 43.088813 32.839756) (width 0.25) (layer B.Cu) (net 2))
 (segment (start 43.088813 32.839756) (end 43.077662 32.806002) (width 0.25) (layer B.Cu) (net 2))
 (segment (start 43.077662 32.806002) (end 43.064868 32.772835) (width 0.25) (layer B.Cu) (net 2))
 (segment (start 43.064868 32.772835) (end 43.050462 32.740336) (width 0.25) (layer B.Cu) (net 2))
 (segment (start 43.050462 32.740336) (end 43.034479 32.708583) (width 0.25) (layer B.Cu) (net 2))
 (segment (start 43.034479 32.708583) (end 43.016957 32.677652) (width 0.25) (layer B.Cu) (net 2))
 (segment (start 43.016957 32.677652) (end 42.997939 32.647619) (width 0.25) (layer B.Cu) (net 2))
 (segment (start 42.997939 32.647619) (end 42.977469 32.618555) (width 0.25) (layer B.Cu) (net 2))
 (segment (start 42.977469 32.618555) (end 42.955599 32.59053) (width 0.25) (layer B.Cu) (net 2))
 (segment (start 42.955599 32.59053) (end 42.932379 32.563612) (width 0.25) (layer B.Cu) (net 2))
 (segment (start 42.932379 32.563612) (end 42.907867 32.537867) (width 0.25) (layer B.Cu) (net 2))
 (segment (start 42.907867 32.537867) (end 42.652132 32.282132) (width 0.25) (layer B.Cu) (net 2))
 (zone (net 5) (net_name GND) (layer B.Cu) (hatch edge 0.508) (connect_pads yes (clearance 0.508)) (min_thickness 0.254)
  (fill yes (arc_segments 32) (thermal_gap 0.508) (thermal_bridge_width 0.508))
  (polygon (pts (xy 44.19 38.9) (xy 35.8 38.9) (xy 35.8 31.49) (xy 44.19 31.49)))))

